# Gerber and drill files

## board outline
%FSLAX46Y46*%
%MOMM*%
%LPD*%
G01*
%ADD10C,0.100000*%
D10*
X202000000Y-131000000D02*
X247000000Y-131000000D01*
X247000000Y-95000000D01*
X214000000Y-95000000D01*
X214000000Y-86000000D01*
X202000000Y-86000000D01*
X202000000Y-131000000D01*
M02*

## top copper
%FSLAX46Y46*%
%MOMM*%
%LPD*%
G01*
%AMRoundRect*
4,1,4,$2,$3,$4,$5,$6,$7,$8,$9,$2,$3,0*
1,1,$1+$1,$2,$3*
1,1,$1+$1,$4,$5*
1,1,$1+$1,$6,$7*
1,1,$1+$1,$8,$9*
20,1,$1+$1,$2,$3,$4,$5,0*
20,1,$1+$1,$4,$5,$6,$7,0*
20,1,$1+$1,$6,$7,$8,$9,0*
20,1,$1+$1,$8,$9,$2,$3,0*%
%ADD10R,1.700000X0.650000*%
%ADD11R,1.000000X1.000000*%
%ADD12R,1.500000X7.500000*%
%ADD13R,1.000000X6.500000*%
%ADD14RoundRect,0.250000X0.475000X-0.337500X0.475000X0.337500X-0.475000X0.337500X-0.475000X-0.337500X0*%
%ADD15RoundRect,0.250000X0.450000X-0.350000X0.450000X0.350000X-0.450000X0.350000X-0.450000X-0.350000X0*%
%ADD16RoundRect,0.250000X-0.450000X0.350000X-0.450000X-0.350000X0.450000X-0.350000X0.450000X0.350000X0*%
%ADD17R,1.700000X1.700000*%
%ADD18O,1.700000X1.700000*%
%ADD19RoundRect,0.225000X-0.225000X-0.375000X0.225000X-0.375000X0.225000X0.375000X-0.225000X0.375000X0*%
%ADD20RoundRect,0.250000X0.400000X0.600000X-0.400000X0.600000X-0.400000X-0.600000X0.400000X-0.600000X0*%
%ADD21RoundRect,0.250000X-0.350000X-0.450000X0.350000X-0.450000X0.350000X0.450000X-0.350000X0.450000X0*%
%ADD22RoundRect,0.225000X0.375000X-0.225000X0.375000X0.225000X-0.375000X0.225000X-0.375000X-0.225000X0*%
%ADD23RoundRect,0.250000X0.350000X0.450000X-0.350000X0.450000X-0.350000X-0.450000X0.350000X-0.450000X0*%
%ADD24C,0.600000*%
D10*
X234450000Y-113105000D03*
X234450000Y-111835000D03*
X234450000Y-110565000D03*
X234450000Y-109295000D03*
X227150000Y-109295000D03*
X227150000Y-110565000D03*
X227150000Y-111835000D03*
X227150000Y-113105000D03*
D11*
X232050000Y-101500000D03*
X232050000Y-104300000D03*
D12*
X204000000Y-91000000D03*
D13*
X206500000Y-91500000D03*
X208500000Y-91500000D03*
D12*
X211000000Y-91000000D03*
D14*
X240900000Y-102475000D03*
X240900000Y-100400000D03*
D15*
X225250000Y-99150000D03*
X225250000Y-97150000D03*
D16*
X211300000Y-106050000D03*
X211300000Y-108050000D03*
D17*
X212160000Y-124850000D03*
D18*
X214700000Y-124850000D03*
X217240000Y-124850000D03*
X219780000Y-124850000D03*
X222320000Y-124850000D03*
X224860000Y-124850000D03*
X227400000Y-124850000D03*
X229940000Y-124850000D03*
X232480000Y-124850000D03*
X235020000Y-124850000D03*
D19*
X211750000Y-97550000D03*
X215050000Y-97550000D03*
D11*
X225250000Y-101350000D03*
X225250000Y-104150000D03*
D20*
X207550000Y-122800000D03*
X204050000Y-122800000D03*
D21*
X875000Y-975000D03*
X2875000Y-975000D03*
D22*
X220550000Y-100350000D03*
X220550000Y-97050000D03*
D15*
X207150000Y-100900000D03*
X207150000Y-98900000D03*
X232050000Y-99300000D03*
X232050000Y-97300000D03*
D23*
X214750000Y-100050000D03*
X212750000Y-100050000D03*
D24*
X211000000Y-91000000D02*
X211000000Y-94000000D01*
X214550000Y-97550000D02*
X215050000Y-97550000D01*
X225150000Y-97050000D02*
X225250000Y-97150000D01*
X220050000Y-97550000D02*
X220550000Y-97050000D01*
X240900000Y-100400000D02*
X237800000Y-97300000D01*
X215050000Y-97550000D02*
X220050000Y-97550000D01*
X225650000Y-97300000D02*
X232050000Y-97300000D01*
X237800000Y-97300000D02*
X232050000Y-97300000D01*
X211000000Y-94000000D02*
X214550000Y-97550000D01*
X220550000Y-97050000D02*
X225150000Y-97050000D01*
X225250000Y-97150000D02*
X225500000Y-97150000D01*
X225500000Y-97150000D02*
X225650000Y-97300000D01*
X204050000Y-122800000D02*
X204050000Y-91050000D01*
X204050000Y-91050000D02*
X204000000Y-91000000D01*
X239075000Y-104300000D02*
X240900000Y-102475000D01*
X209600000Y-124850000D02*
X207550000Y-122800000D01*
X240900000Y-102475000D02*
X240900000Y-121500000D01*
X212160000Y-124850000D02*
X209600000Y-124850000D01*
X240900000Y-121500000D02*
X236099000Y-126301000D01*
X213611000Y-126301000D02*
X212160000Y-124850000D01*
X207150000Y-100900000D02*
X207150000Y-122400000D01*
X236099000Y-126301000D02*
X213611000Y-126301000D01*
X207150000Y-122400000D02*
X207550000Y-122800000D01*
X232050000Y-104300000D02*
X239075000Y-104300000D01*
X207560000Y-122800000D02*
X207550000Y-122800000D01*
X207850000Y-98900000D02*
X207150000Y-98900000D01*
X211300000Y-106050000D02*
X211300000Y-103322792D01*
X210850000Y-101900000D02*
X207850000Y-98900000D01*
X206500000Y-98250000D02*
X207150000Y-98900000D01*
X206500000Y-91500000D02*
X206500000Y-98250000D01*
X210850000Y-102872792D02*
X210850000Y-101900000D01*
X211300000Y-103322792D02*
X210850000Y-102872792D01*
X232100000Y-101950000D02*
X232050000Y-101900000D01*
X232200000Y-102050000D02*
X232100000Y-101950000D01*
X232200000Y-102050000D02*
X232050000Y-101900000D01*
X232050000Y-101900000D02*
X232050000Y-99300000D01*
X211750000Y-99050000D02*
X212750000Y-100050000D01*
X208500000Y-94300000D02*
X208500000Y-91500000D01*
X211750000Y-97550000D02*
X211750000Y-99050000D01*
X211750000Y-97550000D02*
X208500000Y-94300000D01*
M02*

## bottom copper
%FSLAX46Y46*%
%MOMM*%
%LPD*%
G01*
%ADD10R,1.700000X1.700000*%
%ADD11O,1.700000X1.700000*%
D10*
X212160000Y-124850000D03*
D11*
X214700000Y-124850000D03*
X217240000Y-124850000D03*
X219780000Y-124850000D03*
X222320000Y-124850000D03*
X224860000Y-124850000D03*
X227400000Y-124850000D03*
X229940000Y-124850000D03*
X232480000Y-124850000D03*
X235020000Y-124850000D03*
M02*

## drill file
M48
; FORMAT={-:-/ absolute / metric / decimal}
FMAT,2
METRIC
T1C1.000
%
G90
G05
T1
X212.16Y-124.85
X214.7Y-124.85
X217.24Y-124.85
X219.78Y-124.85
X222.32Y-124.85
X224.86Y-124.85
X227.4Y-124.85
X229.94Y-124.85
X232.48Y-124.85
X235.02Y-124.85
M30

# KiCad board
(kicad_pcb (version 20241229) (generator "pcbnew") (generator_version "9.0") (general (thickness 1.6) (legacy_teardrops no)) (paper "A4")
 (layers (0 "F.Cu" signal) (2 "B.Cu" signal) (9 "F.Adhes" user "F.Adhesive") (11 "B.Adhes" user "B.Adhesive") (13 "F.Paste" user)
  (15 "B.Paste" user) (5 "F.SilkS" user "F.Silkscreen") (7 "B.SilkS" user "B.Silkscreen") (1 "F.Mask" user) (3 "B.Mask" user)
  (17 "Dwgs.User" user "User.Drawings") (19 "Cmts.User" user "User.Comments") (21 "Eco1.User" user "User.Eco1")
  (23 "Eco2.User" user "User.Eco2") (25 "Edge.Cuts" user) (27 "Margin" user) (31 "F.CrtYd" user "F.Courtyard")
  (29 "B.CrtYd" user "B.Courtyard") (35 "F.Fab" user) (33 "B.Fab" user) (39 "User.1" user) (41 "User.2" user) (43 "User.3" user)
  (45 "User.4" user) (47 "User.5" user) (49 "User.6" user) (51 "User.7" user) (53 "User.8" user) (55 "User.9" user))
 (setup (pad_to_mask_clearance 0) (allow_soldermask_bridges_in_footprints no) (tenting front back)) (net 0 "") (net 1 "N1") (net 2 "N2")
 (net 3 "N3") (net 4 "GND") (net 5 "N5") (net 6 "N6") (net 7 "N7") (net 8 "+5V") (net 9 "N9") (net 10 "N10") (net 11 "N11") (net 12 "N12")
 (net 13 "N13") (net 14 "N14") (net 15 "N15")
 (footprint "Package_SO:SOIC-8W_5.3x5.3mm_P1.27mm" (layer "F.Cu") (at 230.8 111.2 180)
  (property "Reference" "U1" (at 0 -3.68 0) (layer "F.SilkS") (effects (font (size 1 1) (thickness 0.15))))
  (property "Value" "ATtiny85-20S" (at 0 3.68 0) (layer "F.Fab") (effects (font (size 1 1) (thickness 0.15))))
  (pad "1" smd rect (at -3.65 -1.905 180) (size 1.7 0.65) (layers "F.Cu" "F.Mask" "F.Paste") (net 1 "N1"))
  (pad "2" smd rect (at -3.65 -0.635 180) (size 1.7 0.65) (layers "F.Cu" "F.Mask" "F.Paste") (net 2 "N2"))
  (pad "3" smd rect (at -3.65 0.635 180) (size 1.7 0.65) (layers "F.Cu" "F.Mask" "F.Paste") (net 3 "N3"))
  (pad "4" smd rect (at -3.65 1.905 180) (size 1.7 0.65) (layers "F.Cu" "F.Mask" "F.Paste") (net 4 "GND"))
  (pad "5" smd rect (at 3.65 1.905 180) (size 1.7 0.65) (layers "F.Cu" "F.Mask" "F.Paste") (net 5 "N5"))
  (pad "6" smd rect (at 3.65 0.635 180) (size 1.7 0.65) (layers "F.Cu" "F.Mask" "F.Paste") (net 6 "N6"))
  (pad "7" smd rect (at 3.65 -0.635 180) (size 1.7 0.65) (layers "F.Cu" "F.Mask" "F.Paste") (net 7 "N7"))
  (pad "8" smd rect (at 3.65 -1.905 180) (size 1.7 0.65) (layers "F.Cu" "F.Mask" "F.Paste") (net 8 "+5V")))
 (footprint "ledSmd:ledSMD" (layer "F.Cu") (at 232.05 103.3 -90)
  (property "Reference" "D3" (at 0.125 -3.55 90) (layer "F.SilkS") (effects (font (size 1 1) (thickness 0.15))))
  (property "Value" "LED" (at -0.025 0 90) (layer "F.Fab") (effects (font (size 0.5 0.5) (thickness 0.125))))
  (pad "1" smd rect (at -1.8 0 270) (size 1 1) (layers "F.Cu" "F.Mask" "F.Paste") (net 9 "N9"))
  (pad "2" smd rect (at 1 0 270) (size 1 1) (layers "F.Cu" "F.Mask" "F.Paste") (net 8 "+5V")))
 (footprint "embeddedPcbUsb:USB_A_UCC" (layer "F.Cu") (at 207.5 91.2 -90)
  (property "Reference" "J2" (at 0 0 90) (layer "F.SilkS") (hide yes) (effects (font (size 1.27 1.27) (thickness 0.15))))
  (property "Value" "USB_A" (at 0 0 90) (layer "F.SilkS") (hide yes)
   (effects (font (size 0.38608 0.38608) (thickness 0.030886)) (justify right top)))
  (pad "1" smd rect (at -0.2 3.5 270) (size 7.5 1.5) (layers "F.Cu" "F.Mask" "F.Paste") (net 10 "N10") (solder_mask_margin 0.1016))
  (pad "2" smd rect (at 0.3 1 270) (size 6.5 1) (layers "F.Cu" "F.Mask" "F.Paste") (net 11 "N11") (solder_mask_margin 0.1016))
  (pad "3" smd rect (at 0.3 -1 270) (size 6.5 1) (layers "F.Cu" "F.Mask" "F.Paste") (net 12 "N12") (solder_mask_margin 0.1016))
  (pad "4" smd rect (at -0.2 -3.5 270) (size 7.5 1.5) (layers "F.Cu" "F.Mask" "F.Paste") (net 4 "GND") (solder_mask_margin 0.1016)))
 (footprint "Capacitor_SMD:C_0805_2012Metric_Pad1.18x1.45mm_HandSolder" (layer "F.Cu") (at 240.9 101.4375 90)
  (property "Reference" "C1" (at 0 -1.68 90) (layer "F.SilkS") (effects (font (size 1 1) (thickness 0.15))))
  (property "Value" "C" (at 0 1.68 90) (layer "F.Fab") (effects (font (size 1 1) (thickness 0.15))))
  (pad "1" smd roundrect (at -1.0375 0 90) (size 1.175 1.45) (layers "F.Cu" "F.Mask" "F.Paste") (roundrect_rratio 0.212766) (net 8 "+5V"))
  (pad "2" smd roundrect (at 1.0375 0 90) (size 1.175 1.45) (layers "F.Cu" "F.Mask" "F.Paste") (roundrect_rratio 0.212766) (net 4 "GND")))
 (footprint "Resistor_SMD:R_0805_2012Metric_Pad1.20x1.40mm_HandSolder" (layer "F.Cu") (at 225.25 98.15 90)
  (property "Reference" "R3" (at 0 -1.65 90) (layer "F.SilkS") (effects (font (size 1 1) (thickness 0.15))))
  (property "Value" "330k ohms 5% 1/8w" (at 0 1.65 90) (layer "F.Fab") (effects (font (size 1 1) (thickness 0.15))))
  (pad "1" smd roundrect (at -1 0 90) (size 1.2 1.4) (layers "F.Cu" "F.Mask" "F.Paste") (roundrect_rratio 0.208333) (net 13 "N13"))
  (pad "2" smd roundrect (at 1 0 90) (size 1.2 1.4) (layers "F.Cu" "F.Mask" "F.Paste") (roundrect_rratio 0.208333) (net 4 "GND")))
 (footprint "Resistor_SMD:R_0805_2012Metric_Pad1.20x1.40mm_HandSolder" (layer "F.Cu") (at 211.3 107.05 -90)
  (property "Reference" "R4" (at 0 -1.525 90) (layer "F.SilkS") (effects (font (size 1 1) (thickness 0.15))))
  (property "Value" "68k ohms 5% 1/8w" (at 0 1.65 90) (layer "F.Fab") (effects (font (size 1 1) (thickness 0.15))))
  (pad "1" smd roundrect (at -1 0 270) (size 1.2 1.4) (layers "F.Cu" "F.Mask" "F.Paste") (roundrect_rratio 0.208333) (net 11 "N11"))
  (pad "2" smd roundrect (at 1 0 270) (size 1.2 1.4) (layers "F.Cu" "F.Mask" "F.Paste") (roundrect_rratio 0.208333) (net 2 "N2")))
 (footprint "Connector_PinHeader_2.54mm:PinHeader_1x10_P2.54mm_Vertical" (layer "F.Cu") (at 212.16 124.85 90)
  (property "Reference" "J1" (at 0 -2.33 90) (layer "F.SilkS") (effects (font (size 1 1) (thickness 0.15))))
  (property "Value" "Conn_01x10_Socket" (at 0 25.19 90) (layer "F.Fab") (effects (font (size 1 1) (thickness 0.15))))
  (pad "1" thru_hole rect (at 0 0 90) (size 1.7 1.7) (drill 1) (layers "*.Cu" "*.Mask") (remove_unused_layers no) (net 8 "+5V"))
  (pad "2" thru_hole oval (at 0 2.54 90) (size 1.7 1.7) (drill 1) (layers "*.Cu" "*.Mask") (remove_unused_layers no) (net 4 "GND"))
  (pad "3" thru_hole oval (at 0 5.08 90) (size 1.7 1.7) (drill 1) (layers "*.Cu" "*.Mask") (remove_unused_layers no) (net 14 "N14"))
  (pad "4" thru_hole oval (at 0 7.62 90) (size 1.7 1.7) (drill 1) (layers "*.Cu" "*.Mask") (remove_unused_layers no) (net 5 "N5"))
  (pad "5" thru_hole oval (at 0 10.16 90) (size 1.7 1.7) (drill 1) (layers "*.Cu" "*.Mask") (remove_unused_layers no) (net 6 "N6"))
  (pad "6" thru_hole oval (at 0 12.7 90) (size 1.7 1.7) (drill 1) (layers "*.Cu" "*.Mask") (remove_unused_layers no) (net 7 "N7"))
  (pad "7" thru_hole oval (at 0 15.24 90) (size 1.7 1.7) (drill 1) (layers "*.Cu" "*.Mask") (remove_unused_layers no) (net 2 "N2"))
  (pad "8" thru_hole oval (at 0 17.78 90) (size 1.7 1.7) (drill 1) (layers "*.Cu" "*.Mask") (remove_unused_layers no) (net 3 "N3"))
  (pad "9" thru_hole oval (at 0 20.32 90) (size 1.7 1.7) (drill 1) (layers "*.Cu" "*.Mask") (remove_unused_layers no) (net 1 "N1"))
  (pad "10" thru_hole oval (at 0 22.86 90) (size 1.7 1.7) (drill 1) (layers "*.Cu" "*.Mask") (remove_unused_layers no) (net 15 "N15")))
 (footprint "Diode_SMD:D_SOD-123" (layer "F.Cu") (at 213.4 97.55)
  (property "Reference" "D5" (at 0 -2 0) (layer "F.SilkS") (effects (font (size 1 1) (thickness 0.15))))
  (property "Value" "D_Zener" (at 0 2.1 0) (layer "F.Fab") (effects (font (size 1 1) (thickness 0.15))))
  (pad "1" smd roundrect (at -1.65 0) (size 0.9 1.2) (layers "F.Cu" "F.Mask" "F.Paste") (roundrect_rratio 0.25) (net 12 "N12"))
  (pad "2" smd roundrect (at 1.65 0) (size 0.9 1.2) (layers "F.Cu" "F.Mask" "F.Paste") (roundrect_rratio 0.25) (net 4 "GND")))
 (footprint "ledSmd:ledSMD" (layer "F.Cu") (at 225.25 103.15 -90)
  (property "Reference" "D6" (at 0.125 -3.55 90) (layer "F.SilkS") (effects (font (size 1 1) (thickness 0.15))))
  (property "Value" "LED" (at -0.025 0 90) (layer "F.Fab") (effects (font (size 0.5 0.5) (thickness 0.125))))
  (pad "1" smd rect (at -1.8 0 270) (size 1 1) (layers "F.Cu" "F.Mask" "F.Paste") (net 13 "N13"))
  (pad "2" smd rect (at 1 0 270) (size 1 1) (layers "F.Cu" "F.Mask" "F.Paste") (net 6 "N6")))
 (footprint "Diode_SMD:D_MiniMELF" (layer "F.Cu") (at 205.8 122.8 180)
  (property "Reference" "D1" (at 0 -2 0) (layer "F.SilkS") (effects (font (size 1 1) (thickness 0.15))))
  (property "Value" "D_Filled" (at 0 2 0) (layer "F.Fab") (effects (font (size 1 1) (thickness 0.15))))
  (pad "1" smd roundrect (at -1.75 0 180) (size 1.3 1.7) (layers "F.Cu" "F.Mask" "F.Paste") (roundrect_rratio 0.1923076923) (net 8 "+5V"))
  (pad "2" smd roundrect (at 1.75 0 180) (size 1.3 1.7) (layers "F.Cu" "F.Mask" "F.Paste") (roundrect_rratio 0.1923076923) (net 10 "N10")))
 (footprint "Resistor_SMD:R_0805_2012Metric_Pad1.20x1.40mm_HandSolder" (layer "F.Cu") (at 1.875 0.975)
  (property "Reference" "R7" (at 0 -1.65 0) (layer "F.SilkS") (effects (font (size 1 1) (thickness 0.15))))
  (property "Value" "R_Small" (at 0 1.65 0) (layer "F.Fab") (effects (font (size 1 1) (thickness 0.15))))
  (pad "1" smd roundrect (at -1 0) (size 1.2 1.4) (layers "F.Cu" "F.Mask" "F.Paste") (roundrect_rratio 0.208333))
  (pad "2" smd roundrect (at 1 0) (size 1.2 1.4) (layers "F.Cu" "F.Mask" "F.Paste") (roundrect_rratio 0.208333)))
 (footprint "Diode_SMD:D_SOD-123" (layer "F.Cu") (at 220.55 98.7 90)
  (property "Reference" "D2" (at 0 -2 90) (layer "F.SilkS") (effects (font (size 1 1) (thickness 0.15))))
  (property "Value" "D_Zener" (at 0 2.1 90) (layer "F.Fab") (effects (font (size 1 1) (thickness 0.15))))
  (pad "1" smd roundrect (at -1.65 0 90) (size 0.9 1.2) (layers "F.Cu" "F.Mask" "F.Paste") (roundrect_rratio 0.25) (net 11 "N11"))
  (pad "2" smd roundrect (at 1.65 0 90) (size 0.9 1.2) (layers "F.Cu" "F.Mask" "F.Paste") (roundrect_rratio 0.25) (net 4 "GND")))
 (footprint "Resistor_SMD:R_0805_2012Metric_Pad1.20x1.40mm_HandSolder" (layer "F.Cu") (at 207.15 99.9 90)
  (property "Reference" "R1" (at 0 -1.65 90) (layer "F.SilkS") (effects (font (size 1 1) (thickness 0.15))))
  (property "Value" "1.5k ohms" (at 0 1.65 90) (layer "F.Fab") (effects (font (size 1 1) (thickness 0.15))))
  (pad "1" smd roundrect (at -1 0 90) (size 1.2 1.4) (layers "F.Cu" "F.Mask" "F.Paste") (roundrect_rratio 0.208333) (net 8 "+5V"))
  (pad "2" smd roundrect (at 1 0 90) (size 1.2 1.4) (layers "F.Cu" "F.Mask" "F.Paste") (roundrect_rratio 0.208333) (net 11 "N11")))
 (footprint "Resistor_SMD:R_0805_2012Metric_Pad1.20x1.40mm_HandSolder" (layer "F.Cu") (at 232.05 98.3 90)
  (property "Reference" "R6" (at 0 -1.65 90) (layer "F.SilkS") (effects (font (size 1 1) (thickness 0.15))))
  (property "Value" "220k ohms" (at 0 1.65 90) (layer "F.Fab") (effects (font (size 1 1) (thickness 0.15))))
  (pad "1" smd roundrect (at -1 0 90) (size 1.2 1.4) (layers "F.Cu" "F.Mask" "F.Paste") (roundrect_rratio 0.208333) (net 9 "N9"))
  (pad "2" smd roundrect (at 1 0 90) (size 1.2 1.4) (layers "F.Cu" "F.Mask" "F.Paste") (roundrect_rratio 0.208333) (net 4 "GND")))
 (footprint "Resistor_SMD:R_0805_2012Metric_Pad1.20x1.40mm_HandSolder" (layer "F.Cu") (at 213.75 100.05 180)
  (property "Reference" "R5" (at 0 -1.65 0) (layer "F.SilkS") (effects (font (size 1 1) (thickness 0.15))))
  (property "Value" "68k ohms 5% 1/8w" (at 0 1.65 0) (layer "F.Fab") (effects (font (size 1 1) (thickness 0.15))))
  (pad "1" smd roundrect (at -1 0 180) (size 1.2 1.4) (layers "F.Cu" "F.Mask" "F.Paste") (roundrect_rratio 0.208333) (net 3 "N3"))
  (pad "2" smd roundrect (at 1 0 180) (size 1.2 1.4) (layers "F.Cu" "F.Mask" "F.Paste") (roundrect_rratio 0.208333) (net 12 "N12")))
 (gr_poly
  (pts (xy 202 131) (xy 247 131) (xy 247 95) (xy 214 95) (xy 214 86) (xy 202 86)) (stroke (width 0.1) (type solid)) (fill no)
  (layer "Edge.Cuts"))
 (segment (start 211 91) (end 211 94) (width 0.6) (layer "F.Cu") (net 4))
 (segment (start 214.55 97.55) (end 215.05 97.55) (width 0.6) (layer "F.Cu") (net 4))
 (segment (start 225.15 97.05) (end 225.25 97.15) (width 0.6) (layer "F.Cu") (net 4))
 (segment (start 220.05 97.55) (end 220.55 97.05) (width 0.6) (layer "F.Cu") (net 4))
 (segment (start 240.9 100.4) (end 237.8 97.3) (width 0.6) (layer "F.Cu") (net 4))
 (segment (start 215.05 97.55) (end 220.05 97.55) (width 0.6) (layer "F.Cu") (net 4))
 (segment (start 225.65 97.3) (end 232.05 97.3) (width 0.6) (layer "F.Cu") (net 4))
 (segment (start 237.8 97.3) (end 232.05 97.3) (width 0.6) (layer "F.Cu") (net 4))
 (segment (start 211 94) (end 214.55 97.55) (width 0.6) (layer "F.Cu") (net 4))
 (segment (start 220.55 97.05) (end 225.15 97.05) (width 0.6) (layer "F.Cu") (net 4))
 (segment (start 225.25 97.15) (end 225.5 97.15) (width 0.6) (layer "F.Cu") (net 4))
 (segment (start 225.5 97.15) (end 225.65 97.3) (width 0.6) (layer "F.Cu") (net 4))
 (segment (start 204.05 122.8) (end 204.05 91.05) (width 0.6) (layer "F.Cu") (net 10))
 (segment (start 204.05 91.05) (end 204 91) (width 0.6) (layer "F.Cu") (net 10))
 (segment (start 239.075 104.3) (end 240.9 102.475) (width 0.6) (layer "F.Cu") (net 8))
 (segment (start 209.6 124.85) (end 207.55 122.8) (width 0.6) (layer "F.Cu") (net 8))
 (segment (start 240.9 102.475) (end 240.9 121.5) (width 0.6) (layer "F.Cu") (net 8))
 (segment (start 212.16 124.85) (end 209.6 124.85) (width 0.6) (layer "F.Cu") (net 8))
 (segment (start 240.9 121.5) (end 236.099 126.301) (width 0.6) (layer "F.Cu") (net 8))
 (segment (start 213.611 126.301) (end 212.16 124.85) (width 0.6) (layer "F.Cu") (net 8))
 (segment (start 207.15 100.9) (end 207.15 122.4) (width 0.6) (layer "F.Cu") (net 8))
 (segment (start 236.099 126.301) (end 213.611 126.301) (width 0.6) (layer "F.Cu") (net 8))
 (segment (start 207.15 122.4) (end 207.55 122.8) (width 0.6) (layer "F.Cu") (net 8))
 (segment (start 232.05 104.3) (end 239.075 104.3) (width 0.6) (layer "F.Cu") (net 8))
 (segment (start 207.56 122.8) (end 207.55 122.8) (width 0.6) (layer "F.Cu") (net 8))
 (segment (start 207.85 98.9) (end 207.15 98.9) (width 0.6) (layer "F.Cu") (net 11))
 (segment (start 211.3 106.05) (end 211.3 103.322792) (width 0.6) (layer "F.Cu") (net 11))
 (segment (start 210.85 101.9) (end 207.85 98.9) (width 0.6) (layer "F.Cu") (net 11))
 (segment (start 206.5 98.25) (end 207.15 98.9) (width 0.6) (layer "F.Cu") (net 11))
 (segment (start 206.5 91.5) (end 206.5 98.25) (width 0.6) (layer "F.Cu") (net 11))
 (segment (start 210.85 102.872792) (end 210.85 101.9) (width 0.6) (layer "F.Cu") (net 11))
 (segment (start 211.3 103.322792) (end 210.85 102.872792) (width 0.6) (layer "F.Cu") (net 11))
 (segment (start 232.1 101.95) (end 232.05 101.9) (width 0.6) (layer "F.Cu") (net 9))
 (segment (start 232.2 102.05) (end 232.1 101.95) (width 0.6) (layer "F.Cu") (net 9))
 (segment (start 232.2 102.05) (end 232.05 101.9) (width 0.6) (layer "F.Cu") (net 9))
 (segment (start 232.05 101.9) (end 232.05 99.3) (width 0.6) (layer "F.Cu") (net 9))
 (segment (start 211.75 99.05) (end 212.75 100.05) (width 0.6) (layer "F.Cu") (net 12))
 (segment (start 208.5 94.3) (end 208.5 91.5) (width 0.6) (layer "F.Cu") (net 12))
 (segment (start 211.75 97.55) (end 211.75 99.05) (width 0.6) (layer "F.Cu") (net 12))
 (segment (start 211.75 97.55) (end 208.5 94.3) (width 0.6) (layer "F.Cu") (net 12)))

